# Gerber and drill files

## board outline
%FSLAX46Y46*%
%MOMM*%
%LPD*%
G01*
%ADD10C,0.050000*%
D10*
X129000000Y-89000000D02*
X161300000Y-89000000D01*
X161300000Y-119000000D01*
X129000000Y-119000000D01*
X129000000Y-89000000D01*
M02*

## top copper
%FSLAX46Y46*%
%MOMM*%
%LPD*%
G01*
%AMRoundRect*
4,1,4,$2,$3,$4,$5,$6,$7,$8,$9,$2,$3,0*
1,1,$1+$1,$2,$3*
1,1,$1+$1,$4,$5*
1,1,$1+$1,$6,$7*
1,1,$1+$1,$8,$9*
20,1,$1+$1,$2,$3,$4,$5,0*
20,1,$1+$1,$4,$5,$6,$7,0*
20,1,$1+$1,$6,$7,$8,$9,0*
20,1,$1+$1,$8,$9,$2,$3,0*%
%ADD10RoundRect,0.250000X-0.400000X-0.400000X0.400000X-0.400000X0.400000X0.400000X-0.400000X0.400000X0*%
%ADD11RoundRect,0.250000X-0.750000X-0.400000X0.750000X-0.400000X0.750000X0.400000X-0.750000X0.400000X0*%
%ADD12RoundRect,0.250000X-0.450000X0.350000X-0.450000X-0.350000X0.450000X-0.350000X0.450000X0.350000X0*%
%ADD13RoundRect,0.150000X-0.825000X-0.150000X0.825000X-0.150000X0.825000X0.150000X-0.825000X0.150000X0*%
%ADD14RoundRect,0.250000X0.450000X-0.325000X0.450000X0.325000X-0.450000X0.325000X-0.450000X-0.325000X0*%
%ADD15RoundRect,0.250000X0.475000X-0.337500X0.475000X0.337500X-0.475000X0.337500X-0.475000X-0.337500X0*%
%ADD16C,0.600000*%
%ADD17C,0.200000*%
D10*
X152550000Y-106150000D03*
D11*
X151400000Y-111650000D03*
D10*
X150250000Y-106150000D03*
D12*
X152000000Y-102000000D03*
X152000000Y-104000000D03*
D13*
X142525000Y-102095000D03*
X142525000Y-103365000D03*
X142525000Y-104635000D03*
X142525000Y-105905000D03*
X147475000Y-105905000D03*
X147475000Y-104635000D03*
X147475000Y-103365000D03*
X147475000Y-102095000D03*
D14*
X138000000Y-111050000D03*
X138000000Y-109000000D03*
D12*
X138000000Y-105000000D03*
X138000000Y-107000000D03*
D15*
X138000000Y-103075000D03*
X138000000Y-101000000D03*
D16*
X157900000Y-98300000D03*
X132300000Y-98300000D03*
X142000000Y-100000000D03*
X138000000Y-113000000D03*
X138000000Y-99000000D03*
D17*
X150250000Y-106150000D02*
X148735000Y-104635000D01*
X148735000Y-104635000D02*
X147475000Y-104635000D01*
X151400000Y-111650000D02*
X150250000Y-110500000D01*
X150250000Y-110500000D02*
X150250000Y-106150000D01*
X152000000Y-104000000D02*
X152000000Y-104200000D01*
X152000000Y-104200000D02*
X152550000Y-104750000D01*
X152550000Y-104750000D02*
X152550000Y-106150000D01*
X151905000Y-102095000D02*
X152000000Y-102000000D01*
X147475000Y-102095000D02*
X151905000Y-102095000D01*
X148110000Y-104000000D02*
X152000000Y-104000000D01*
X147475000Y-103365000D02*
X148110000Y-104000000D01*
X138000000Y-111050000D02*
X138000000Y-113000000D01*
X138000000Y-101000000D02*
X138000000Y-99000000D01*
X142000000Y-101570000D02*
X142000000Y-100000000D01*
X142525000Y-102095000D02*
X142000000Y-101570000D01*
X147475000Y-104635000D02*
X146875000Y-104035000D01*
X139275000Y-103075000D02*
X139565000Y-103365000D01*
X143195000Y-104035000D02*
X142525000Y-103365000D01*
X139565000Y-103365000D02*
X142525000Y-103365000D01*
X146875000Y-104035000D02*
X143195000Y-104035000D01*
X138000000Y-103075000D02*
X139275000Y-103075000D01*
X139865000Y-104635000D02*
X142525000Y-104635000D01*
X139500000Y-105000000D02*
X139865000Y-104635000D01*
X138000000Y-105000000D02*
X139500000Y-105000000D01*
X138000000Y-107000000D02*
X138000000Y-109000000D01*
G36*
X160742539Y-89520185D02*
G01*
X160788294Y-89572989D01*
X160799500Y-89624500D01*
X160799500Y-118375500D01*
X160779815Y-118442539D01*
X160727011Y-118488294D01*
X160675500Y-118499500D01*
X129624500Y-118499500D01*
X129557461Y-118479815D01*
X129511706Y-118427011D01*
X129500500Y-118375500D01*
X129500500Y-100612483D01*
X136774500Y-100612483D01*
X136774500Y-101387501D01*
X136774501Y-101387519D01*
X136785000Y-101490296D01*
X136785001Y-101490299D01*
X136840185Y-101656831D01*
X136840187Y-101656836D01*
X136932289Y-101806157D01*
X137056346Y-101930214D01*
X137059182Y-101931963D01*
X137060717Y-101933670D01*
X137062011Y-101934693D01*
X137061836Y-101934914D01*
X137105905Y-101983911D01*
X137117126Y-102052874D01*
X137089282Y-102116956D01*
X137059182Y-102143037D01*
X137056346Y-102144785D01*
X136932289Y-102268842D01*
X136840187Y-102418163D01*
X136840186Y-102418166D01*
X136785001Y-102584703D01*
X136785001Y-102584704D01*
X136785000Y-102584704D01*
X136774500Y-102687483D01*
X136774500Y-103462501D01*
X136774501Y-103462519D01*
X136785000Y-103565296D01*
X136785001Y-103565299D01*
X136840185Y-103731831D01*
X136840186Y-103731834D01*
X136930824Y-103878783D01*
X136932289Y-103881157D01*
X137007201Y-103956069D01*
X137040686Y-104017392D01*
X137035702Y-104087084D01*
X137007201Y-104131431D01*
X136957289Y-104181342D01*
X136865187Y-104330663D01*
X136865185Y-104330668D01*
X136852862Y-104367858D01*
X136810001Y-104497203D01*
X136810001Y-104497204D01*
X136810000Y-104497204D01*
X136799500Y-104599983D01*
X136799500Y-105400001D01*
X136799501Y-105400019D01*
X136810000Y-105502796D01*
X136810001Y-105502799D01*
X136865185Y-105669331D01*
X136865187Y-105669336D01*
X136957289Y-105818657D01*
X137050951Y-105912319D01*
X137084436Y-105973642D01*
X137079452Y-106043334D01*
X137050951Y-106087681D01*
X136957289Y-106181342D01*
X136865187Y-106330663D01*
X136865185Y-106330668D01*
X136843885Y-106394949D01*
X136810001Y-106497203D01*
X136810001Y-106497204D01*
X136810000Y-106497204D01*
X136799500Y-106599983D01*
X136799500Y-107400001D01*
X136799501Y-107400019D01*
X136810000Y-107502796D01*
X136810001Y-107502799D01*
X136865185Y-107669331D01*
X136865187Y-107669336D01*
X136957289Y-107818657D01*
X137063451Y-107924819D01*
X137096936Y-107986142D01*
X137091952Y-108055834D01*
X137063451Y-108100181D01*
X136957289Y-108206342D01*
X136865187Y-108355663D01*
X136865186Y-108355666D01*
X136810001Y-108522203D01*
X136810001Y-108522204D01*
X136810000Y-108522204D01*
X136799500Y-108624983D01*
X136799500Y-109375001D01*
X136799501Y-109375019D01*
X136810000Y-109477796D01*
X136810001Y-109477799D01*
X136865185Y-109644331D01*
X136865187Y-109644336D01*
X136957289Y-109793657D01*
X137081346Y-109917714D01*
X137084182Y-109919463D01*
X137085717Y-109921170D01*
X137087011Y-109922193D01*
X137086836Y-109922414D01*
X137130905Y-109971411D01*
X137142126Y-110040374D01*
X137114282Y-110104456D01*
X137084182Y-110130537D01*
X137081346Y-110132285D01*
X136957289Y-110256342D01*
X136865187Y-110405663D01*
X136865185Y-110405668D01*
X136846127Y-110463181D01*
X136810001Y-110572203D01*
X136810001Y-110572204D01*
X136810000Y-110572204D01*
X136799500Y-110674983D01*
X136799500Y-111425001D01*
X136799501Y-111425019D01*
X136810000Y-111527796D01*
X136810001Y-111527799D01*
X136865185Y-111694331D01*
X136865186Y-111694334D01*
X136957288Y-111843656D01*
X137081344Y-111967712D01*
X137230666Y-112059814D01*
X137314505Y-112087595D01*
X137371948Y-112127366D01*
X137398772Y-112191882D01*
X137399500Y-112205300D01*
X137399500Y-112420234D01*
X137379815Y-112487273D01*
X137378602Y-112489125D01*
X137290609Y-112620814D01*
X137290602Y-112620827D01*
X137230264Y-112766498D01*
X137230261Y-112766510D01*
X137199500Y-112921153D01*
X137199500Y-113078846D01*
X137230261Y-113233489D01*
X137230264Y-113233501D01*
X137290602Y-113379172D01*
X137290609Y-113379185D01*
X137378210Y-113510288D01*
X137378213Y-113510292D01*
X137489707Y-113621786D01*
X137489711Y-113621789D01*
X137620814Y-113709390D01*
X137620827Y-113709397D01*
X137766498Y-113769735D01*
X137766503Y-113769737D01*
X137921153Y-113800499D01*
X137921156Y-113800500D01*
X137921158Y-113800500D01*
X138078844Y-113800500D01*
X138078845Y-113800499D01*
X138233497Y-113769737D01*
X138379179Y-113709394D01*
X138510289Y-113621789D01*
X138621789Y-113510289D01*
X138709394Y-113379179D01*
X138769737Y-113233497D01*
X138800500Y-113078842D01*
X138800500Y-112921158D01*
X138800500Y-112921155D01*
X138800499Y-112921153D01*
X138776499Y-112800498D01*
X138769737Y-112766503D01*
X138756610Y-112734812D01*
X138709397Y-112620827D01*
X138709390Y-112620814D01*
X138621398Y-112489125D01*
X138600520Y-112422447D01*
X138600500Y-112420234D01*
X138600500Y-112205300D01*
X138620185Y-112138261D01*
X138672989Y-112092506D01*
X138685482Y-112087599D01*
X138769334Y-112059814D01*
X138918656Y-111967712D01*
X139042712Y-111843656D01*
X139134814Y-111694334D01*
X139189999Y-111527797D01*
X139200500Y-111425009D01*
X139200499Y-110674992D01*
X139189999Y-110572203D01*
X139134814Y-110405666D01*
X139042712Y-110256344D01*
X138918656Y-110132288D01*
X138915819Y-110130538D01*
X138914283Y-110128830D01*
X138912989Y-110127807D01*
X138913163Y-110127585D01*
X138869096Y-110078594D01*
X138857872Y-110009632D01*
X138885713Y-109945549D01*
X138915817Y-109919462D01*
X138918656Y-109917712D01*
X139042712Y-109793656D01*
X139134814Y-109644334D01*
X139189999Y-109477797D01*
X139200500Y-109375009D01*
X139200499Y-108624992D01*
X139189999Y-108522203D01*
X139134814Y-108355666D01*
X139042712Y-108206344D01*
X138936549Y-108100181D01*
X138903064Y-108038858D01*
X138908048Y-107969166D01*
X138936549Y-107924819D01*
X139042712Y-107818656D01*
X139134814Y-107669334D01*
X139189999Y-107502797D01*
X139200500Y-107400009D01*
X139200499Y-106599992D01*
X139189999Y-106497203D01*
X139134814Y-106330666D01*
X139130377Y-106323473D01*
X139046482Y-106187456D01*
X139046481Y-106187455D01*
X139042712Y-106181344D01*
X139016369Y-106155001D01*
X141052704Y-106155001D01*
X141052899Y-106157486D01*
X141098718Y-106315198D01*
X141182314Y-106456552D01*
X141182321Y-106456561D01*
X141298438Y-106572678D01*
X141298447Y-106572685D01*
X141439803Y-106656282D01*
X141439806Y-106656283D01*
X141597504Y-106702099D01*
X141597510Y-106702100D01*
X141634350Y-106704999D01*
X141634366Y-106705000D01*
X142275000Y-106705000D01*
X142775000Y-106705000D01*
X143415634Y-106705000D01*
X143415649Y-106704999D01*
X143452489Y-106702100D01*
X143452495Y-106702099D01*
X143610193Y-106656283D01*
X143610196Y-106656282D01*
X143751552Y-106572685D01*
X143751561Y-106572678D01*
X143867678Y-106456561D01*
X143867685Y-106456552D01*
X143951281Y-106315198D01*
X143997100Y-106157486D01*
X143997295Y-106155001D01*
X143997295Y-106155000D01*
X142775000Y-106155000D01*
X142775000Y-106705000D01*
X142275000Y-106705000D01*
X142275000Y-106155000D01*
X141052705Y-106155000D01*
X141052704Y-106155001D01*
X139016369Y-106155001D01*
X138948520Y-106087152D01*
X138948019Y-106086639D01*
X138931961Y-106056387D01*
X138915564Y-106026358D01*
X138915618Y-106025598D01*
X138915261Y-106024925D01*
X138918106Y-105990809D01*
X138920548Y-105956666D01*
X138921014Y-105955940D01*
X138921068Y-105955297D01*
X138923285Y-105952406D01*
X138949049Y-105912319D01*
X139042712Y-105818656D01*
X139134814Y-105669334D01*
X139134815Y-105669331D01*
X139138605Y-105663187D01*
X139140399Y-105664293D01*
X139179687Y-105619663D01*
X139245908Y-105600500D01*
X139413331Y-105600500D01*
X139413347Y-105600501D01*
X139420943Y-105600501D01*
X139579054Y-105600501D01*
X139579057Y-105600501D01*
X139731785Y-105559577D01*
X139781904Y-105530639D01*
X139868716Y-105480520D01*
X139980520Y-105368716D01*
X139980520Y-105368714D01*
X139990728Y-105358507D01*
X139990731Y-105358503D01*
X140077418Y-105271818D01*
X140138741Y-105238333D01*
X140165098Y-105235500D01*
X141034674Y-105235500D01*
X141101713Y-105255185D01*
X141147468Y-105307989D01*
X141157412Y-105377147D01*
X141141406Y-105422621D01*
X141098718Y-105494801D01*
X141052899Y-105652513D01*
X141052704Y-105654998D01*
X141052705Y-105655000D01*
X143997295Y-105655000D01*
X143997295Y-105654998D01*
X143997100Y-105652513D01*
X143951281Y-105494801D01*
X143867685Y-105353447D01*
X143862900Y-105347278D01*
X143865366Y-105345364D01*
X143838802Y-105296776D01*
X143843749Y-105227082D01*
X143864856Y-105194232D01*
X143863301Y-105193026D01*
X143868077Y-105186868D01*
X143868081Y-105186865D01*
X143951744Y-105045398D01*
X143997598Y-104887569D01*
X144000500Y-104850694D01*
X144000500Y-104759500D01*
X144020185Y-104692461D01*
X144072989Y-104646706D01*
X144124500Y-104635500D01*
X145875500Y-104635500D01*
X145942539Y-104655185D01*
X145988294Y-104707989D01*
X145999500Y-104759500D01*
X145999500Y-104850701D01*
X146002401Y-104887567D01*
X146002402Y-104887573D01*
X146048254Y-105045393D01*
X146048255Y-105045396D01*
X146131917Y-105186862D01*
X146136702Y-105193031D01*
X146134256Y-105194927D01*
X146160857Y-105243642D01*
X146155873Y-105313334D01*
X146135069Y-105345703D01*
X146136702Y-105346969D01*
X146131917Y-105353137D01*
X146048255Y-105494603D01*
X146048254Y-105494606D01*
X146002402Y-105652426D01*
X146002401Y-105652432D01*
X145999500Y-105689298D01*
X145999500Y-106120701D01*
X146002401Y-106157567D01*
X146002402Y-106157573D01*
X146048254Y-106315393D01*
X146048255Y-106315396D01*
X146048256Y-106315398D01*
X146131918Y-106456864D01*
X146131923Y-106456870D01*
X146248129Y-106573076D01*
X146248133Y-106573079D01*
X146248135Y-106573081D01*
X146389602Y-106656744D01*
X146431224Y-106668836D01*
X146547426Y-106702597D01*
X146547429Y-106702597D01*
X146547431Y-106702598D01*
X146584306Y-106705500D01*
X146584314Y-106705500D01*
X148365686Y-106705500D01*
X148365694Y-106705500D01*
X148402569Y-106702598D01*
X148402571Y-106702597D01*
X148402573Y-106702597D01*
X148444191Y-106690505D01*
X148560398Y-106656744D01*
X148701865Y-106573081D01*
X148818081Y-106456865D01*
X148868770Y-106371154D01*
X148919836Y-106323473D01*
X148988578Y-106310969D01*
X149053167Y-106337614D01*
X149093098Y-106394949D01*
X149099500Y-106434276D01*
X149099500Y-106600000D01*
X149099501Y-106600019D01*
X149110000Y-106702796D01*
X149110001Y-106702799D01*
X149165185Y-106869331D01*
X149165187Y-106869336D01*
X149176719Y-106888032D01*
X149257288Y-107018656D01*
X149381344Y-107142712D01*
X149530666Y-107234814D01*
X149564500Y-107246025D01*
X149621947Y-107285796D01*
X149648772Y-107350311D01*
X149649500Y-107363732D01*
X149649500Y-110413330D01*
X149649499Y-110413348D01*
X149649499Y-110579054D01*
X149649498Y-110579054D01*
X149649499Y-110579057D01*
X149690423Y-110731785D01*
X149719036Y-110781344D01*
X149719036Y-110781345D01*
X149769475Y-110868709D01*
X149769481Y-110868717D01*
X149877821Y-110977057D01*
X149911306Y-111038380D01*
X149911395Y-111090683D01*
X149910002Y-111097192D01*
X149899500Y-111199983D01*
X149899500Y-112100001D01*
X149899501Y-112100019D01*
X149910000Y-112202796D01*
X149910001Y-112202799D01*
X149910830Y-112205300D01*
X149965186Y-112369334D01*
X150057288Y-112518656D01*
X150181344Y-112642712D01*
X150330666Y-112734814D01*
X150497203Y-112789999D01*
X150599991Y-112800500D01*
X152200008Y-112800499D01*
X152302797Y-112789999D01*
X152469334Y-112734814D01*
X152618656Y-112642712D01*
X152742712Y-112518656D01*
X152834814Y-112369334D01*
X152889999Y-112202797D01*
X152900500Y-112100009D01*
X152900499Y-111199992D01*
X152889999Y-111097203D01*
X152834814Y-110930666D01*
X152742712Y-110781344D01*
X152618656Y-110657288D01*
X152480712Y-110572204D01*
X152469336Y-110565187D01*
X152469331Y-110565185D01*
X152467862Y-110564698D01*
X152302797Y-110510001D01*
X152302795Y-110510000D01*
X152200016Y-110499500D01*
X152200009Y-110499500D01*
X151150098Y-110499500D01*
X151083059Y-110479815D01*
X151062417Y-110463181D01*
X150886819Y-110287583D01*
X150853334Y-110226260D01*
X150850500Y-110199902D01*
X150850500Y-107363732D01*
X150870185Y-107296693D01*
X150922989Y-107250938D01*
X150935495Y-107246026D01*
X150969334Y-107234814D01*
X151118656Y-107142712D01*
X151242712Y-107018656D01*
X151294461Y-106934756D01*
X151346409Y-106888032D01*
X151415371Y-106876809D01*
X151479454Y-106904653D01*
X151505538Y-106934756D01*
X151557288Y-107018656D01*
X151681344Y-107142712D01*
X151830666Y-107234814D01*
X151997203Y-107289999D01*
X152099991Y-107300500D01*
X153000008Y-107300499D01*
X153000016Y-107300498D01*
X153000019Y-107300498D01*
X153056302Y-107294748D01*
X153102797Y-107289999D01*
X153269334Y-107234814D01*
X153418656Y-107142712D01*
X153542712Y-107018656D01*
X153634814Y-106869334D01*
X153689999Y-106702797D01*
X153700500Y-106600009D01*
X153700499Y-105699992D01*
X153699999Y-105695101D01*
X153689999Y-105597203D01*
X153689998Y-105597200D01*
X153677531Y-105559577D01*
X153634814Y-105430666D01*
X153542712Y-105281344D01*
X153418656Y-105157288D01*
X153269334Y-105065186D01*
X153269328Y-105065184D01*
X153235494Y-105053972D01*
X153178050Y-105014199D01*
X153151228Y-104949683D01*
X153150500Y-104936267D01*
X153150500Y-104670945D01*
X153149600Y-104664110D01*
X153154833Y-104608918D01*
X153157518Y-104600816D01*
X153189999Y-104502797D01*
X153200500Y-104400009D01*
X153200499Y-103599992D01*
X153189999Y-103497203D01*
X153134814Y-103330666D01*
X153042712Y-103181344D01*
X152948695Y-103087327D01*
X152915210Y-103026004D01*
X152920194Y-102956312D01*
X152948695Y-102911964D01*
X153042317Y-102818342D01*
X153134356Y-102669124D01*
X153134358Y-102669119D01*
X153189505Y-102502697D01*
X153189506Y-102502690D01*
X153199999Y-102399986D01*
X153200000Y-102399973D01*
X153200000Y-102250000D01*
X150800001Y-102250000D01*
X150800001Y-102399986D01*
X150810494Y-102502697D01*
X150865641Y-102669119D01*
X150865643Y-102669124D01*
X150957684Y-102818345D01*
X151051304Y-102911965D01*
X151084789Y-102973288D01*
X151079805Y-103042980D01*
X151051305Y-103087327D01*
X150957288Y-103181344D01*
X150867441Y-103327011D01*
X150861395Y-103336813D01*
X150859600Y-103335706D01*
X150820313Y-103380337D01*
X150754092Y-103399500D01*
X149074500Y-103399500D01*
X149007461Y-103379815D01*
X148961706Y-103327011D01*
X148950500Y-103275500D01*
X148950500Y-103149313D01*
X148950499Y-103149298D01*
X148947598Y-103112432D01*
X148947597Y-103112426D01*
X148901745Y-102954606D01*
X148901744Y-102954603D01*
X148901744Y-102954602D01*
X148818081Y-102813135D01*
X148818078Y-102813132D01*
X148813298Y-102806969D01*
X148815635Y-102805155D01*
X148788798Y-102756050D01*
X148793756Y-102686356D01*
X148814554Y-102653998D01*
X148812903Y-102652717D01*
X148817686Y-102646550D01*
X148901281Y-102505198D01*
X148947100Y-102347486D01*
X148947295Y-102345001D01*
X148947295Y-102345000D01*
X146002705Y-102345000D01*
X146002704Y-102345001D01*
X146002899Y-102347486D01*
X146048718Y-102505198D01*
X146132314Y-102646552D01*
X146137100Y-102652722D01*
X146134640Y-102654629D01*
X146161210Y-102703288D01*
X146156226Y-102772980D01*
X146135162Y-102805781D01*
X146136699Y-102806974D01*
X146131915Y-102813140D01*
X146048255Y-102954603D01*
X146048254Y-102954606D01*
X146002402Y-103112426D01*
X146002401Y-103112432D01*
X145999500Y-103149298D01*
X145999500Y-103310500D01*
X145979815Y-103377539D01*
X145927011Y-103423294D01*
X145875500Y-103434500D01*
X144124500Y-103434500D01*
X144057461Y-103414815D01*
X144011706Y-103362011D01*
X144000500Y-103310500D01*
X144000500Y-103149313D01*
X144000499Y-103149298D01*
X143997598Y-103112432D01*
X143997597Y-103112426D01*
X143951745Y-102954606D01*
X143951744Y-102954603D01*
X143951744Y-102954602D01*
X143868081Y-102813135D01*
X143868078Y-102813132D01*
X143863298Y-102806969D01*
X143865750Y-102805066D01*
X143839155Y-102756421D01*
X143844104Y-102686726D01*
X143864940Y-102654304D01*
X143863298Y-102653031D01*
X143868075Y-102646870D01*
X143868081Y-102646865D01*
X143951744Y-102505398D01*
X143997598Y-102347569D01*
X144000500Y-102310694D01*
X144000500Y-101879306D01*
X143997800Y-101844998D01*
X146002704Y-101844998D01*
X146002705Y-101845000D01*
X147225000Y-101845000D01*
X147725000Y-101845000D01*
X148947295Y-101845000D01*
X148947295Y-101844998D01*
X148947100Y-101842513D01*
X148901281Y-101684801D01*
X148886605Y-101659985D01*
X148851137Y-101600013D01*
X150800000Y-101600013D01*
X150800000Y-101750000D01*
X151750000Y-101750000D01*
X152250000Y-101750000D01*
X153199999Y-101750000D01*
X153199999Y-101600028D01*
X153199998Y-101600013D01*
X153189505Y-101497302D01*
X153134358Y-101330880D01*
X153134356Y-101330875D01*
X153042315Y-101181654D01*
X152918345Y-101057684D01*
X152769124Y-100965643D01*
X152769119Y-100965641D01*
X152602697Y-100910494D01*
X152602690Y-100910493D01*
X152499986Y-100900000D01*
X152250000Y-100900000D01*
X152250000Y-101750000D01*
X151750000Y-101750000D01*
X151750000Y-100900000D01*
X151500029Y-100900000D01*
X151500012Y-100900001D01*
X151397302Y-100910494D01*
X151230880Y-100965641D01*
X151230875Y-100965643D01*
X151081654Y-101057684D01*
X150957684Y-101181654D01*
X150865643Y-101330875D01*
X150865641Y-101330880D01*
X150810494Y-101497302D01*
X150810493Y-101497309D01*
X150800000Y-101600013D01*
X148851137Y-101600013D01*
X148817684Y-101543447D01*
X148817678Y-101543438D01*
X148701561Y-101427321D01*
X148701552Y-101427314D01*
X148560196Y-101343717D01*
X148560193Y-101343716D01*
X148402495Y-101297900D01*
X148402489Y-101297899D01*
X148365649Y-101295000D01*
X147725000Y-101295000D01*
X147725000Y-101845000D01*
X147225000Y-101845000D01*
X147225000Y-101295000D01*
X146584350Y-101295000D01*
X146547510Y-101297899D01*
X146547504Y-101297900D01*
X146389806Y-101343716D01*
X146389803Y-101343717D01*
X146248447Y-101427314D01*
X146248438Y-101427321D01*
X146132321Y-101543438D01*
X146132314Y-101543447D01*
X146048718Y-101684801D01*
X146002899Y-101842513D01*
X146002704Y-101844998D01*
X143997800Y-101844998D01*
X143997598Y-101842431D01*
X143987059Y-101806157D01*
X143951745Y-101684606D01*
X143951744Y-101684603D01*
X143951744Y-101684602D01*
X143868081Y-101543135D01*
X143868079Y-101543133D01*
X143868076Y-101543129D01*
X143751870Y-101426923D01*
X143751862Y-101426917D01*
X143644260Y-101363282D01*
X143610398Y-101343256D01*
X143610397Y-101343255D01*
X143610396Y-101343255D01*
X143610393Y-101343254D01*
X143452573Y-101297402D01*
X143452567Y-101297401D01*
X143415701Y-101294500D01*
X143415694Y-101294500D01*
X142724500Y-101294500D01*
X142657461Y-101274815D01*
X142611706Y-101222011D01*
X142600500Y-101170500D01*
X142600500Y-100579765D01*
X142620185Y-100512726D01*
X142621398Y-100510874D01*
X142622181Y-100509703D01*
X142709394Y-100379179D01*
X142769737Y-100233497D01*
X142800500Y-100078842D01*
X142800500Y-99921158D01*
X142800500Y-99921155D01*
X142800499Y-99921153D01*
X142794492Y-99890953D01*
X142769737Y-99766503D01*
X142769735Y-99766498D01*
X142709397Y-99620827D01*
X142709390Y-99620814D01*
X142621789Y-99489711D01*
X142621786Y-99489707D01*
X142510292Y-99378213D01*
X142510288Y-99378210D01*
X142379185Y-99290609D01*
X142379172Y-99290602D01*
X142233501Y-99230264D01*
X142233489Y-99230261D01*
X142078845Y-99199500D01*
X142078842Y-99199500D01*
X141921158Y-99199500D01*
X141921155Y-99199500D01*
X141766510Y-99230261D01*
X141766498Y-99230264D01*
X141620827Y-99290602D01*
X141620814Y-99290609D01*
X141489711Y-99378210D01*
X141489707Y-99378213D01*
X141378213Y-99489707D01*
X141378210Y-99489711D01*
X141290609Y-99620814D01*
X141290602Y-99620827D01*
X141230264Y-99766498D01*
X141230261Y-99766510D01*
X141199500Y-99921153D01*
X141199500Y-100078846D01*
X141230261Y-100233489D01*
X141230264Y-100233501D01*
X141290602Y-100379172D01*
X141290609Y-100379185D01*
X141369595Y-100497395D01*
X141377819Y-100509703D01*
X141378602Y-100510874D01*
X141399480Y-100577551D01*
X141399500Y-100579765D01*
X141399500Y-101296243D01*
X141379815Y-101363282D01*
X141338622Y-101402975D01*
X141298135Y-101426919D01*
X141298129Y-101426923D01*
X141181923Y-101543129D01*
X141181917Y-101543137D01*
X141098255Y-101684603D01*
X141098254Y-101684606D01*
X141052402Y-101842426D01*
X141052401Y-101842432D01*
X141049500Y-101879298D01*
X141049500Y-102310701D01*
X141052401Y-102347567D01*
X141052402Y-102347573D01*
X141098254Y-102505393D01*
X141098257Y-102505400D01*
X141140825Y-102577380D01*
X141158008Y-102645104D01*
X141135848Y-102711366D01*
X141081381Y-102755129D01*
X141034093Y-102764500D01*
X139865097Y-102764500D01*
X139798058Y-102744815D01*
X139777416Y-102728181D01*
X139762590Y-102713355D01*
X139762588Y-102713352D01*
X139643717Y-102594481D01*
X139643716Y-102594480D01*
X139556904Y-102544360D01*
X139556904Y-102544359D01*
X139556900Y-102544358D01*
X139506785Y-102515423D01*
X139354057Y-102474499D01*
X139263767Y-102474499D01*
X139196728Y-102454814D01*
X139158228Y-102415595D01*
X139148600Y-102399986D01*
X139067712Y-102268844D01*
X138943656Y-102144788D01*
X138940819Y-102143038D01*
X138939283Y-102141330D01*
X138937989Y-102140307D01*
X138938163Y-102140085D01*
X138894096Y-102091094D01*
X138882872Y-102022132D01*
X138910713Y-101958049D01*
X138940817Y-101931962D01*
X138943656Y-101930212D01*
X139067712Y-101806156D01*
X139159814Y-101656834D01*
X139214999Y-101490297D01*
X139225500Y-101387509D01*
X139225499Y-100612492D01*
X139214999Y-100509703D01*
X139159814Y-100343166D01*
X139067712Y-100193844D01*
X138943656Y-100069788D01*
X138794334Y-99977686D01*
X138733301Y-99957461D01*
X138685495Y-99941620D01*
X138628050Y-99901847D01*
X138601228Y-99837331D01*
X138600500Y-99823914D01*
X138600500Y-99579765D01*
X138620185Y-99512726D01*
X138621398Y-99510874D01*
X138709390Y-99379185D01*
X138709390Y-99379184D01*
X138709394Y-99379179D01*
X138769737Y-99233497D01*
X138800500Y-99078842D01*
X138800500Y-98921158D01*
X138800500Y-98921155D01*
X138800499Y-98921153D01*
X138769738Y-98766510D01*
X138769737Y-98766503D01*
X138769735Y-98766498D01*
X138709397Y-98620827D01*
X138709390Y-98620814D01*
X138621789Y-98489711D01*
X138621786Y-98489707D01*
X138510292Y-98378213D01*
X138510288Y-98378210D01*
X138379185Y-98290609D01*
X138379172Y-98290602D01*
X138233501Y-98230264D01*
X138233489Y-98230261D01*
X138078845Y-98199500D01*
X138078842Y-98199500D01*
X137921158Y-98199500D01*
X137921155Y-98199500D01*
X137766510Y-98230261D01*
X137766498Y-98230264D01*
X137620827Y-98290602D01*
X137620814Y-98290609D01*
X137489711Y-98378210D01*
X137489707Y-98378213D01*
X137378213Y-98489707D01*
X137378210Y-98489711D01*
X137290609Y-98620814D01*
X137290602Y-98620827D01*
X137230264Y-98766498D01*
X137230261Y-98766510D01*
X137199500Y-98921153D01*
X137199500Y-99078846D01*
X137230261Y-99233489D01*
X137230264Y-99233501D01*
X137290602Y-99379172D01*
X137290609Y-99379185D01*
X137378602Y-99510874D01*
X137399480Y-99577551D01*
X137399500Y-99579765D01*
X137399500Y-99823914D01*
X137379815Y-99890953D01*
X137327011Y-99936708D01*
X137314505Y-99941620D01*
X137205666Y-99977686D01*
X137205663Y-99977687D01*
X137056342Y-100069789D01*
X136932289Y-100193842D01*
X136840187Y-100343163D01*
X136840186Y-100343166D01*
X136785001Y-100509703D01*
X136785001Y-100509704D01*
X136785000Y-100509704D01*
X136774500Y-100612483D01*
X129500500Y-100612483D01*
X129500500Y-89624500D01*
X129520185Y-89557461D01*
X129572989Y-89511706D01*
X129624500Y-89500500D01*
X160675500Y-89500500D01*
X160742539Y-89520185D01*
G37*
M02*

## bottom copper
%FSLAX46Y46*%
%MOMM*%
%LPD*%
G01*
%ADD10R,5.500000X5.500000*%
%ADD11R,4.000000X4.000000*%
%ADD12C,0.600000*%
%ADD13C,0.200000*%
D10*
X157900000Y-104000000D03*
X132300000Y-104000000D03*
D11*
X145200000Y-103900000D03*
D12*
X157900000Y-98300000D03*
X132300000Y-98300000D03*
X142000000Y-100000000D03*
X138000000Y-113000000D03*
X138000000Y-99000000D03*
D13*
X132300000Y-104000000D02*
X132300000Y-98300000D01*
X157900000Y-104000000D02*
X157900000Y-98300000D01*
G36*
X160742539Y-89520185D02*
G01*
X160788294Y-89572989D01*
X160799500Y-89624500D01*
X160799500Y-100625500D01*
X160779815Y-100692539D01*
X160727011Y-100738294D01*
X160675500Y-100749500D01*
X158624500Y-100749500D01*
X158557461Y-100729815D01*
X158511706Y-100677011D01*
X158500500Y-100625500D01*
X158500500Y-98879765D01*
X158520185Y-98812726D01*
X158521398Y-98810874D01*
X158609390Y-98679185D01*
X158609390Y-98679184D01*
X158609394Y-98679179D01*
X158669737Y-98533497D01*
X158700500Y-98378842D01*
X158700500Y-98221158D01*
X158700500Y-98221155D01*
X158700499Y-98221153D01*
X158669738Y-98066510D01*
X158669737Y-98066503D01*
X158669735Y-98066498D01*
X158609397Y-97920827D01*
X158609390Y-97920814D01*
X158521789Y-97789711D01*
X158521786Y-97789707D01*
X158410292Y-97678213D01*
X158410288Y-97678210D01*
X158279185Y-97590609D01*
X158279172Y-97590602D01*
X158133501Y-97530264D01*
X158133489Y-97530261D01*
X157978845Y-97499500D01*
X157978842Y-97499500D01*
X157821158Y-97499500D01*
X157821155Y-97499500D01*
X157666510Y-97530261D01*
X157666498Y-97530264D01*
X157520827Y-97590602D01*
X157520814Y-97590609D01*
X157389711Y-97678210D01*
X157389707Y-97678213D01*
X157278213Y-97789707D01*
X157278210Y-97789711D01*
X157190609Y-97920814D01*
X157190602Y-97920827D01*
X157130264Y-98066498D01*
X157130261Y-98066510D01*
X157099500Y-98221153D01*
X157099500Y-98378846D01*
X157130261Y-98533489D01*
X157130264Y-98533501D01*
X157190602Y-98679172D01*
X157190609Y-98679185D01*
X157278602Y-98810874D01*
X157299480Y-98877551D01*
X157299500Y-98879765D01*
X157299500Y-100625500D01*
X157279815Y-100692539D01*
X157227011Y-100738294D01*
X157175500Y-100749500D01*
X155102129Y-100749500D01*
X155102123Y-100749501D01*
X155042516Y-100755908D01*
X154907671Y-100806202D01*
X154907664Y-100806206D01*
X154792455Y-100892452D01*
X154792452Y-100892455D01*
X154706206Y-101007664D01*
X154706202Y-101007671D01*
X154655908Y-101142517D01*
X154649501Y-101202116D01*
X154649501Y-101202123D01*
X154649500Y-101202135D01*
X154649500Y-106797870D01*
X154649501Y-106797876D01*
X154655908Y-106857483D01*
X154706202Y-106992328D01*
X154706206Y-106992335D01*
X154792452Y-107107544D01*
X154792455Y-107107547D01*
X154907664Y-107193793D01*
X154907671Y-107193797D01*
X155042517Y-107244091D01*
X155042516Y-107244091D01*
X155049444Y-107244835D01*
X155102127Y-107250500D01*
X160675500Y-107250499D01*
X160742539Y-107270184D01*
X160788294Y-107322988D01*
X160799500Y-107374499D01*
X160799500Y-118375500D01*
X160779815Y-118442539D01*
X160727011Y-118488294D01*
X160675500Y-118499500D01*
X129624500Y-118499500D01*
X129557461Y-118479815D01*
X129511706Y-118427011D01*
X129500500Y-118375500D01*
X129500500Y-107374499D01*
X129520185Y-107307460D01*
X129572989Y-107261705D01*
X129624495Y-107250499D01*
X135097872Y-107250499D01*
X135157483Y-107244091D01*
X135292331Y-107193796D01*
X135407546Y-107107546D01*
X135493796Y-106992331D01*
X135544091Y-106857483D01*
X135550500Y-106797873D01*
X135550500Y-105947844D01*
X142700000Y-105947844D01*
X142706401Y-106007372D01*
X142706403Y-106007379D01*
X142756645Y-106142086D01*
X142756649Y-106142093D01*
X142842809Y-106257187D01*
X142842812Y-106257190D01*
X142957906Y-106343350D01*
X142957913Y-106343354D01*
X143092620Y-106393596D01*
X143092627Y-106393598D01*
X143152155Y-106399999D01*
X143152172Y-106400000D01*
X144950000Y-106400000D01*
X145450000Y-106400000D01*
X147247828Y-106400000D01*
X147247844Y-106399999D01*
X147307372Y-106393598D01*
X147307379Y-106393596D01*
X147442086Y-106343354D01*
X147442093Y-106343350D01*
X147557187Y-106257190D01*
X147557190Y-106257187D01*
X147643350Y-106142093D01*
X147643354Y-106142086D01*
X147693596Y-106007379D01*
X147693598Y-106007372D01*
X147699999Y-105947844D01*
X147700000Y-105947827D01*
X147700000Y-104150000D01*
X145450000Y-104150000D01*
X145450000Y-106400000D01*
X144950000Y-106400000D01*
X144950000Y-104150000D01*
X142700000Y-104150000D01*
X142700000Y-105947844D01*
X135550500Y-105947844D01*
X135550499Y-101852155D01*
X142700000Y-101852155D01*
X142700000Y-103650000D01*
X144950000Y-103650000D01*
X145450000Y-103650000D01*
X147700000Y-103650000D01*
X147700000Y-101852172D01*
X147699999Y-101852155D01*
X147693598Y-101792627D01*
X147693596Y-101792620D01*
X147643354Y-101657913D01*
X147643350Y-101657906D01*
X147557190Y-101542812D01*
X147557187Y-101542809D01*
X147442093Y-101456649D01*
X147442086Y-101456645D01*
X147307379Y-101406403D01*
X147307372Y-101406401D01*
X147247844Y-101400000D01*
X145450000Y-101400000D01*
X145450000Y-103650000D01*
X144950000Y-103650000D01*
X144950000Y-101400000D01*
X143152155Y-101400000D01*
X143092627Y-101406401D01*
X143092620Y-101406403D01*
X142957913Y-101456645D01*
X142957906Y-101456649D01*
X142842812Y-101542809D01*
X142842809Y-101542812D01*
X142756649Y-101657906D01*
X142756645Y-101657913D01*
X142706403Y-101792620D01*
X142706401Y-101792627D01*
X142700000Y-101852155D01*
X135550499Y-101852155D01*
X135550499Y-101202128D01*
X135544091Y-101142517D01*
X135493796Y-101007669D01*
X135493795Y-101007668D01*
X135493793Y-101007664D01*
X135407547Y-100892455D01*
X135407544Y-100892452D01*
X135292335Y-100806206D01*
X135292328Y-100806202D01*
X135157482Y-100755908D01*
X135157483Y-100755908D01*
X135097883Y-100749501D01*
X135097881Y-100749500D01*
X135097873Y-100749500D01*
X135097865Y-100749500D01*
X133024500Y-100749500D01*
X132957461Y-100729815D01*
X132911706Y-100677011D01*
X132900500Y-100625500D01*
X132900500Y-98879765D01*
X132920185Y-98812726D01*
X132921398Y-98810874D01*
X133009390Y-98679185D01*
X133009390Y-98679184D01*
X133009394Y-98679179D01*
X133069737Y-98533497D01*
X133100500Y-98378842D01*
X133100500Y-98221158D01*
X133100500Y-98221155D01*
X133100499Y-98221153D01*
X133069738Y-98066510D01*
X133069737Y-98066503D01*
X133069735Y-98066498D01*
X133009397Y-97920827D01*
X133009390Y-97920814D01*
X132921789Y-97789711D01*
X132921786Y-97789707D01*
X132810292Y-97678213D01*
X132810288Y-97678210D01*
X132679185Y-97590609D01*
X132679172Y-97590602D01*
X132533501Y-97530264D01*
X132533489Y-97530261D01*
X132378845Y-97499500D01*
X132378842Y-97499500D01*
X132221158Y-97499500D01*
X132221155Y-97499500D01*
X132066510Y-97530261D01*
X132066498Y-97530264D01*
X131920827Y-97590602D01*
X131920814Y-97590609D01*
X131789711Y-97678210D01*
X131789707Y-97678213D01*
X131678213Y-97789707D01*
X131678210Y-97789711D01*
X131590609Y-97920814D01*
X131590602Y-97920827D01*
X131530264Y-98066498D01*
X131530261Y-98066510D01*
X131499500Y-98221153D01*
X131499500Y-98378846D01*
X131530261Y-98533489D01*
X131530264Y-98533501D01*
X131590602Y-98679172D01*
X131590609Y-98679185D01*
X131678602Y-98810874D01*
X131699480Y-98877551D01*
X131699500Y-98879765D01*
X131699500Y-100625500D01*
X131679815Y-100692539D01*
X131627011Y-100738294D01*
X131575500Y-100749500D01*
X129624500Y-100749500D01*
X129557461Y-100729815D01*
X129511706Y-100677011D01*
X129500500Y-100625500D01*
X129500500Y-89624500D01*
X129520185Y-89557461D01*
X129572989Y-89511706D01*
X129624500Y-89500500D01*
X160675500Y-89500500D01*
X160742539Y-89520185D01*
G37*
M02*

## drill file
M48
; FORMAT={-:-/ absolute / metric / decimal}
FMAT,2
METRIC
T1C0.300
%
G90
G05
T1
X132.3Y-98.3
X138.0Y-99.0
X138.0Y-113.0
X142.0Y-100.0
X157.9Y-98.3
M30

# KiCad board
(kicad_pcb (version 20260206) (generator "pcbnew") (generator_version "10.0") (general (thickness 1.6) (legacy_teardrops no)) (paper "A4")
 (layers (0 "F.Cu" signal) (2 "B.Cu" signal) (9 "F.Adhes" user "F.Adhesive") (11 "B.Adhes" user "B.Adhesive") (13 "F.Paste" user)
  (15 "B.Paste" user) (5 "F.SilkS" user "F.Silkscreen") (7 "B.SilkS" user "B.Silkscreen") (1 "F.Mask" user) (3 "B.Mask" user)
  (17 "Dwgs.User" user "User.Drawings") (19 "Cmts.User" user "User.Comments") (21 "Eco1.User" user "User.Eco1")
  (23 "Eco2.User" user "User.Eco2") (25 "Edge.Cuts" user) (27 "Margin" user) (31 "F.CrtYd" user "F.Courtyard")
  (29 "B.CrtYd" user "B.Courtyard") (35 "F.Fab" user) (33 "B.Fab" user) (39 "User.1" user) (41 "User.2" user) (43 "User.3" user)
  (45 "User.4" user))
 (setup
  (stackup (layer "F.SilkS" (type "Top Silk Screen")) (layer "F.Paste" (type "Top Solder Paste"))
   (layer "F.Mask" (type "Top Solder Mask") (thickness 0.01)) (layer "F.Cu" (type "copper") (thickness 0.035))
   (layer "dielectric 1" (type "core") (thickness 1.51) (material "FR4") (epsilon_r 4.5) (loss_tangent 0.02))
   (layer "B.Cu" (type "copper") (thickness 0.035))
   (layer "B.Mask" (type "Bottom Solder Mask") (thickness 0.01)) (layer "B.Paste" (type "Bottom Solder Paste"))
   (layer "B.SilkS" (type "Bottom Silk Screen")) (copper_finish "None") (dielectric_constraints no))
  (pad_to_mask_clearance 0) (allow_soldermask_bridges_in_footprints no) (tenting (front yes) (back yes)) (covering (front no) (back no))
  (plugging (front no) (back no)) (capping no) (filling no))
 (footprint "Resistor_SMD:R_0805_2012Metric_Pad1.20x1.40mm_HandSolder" (layer "F.Cu") (at 152 103 -90)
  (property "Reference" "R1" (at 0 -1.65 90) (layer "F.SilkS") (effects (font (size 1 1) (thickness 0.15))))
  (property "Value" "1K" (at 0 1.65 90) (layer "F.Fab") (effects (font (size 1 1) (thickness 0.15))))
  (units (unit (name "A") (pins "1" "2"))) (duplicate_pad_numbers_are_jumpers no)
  (pad "1" smd roundrect (at -1 0 270) (size 1.2 1.4) (layers "F.Cu" "F.Mask" "F.Paste") (roundrect_rratio 0.208333) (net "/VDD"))
  (pad "2" smd roundrect (at 1 0 270) (size 1.2 1.4) (layers "F.Cu" "F.Mask" "F.Paste") (roundrect_rratio 0.208333) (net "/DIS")))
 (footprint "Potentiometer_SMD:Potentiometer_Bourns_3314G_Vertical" (layer "F.Cu") (at 151.4 108.9)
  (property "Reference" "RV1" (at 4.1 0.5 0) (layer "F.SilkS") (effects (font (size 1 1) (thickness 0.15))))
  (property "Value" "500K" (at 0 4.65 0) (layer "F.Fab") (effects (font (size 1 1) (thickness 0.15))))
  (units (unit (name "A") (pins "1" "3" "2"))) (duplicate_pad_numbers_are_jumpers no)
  (pad "1" smd roundrect (at 1.15 -2.75) (size 1.3 1.3) (layers "F.Cu" "F.Mask" "F.Paste") (roundrect_rratio 0.192308) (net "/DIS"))
  (pad "2" smd roundrect (at 0 2.75) (size 2 1.3) (layers "F.Cu" "F.Mask" "F.Paste") (roundrect_rratio 0.192308) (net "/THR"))
  (pad "3" smd roundrect (at -1.15 -2.75) (size 1.3 1.3) (layers "F.Cu" "F.Mask" "F.Paste") (roundrect_rratio 0.192308) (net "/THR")))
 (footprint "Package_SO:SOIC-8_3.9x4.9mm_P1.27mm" (layer "F.Cu") (at 145 104)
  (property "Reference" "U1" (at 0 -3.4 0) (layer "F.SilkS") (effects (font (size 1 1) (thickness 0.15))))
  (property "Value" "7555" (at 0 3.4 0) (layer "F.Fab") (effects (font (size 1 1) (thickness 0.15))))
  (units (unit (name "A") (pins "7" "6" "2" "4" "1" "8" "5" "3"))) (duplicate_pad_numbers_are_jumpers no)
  (pad "1" smd roundrect (at -2.475 -1.905) (size 1.95 0.6) (layers "F.Cu" "F.Mask" "F.Paste") (roundrect_rratio 0.25) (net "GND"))
  (pad "2" smd roundrect (at -2.475 -0.635) (size 1.95 0.6) (layers "F.Cu" "F.Mask" "F.Paste") (roundrect_rratio 0.25) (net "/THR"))
  (pad "3" smd roundrect (at -2.475 0.635) (size 1.95 0.6) (layers "F.Cu" "F.Mask" "F.Paste") (roundrect_rratio 0.25) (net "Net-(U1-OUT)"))
  (pad "4" smd roundrect (at -2.475 1.905) (size 1.95 0.6) (layers "F.Cu" "F.Mask" "F.Paste") (roundrect_rratio 0.25) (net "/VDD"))
  (pad "5" smd roundrect (at 2.475 1.905) (size 1.95 0.6) (layers "F.Cu" "F.Mask" "F.Paste") (roundrect_rratio 0.25)
   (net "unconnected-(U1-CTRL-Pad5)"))
  (pad "6" smd roundrect (at 2.475 0.635) (size 1.95 0.6) (layers "F.Cu" "F.Mask" "F.Paste") (roundrect_rratio 0.25) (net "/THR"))
  (pad "7" smd roundrect (at 2.475 -0.635) (size 1.95 0.6) (layers "F.Cu" "F.Mask" "F.Paste") (roundrect_rratio 0.25) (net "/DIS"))
  (pad "8" smd roundrect (at 2.475 -1.905) (size 1.95 0.6) (layers "F.Cu" "F.Mask" "F.Paste") (roundrect_rratio 0.25) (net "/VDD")))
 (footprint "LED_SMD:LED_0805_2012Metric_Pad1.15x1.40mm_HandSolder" (layer "F.Cu") (at 138 110.025 90)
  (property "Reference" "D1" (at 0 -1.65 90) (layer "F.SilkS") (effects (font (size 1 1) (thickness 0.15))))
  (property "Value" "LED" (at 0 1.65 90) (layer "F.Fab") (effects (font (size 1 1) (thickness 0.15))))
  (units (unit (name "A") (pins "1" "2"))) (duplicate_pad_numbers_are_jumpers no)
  (pad "1" smd roundrect (at -1.025 0 90) (size 1.15 1.4) (layers "F.Cu" "F.Mask" "F.Paste") (roundrect_rratio 0.217391) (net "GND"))
  (pad "2" smd roundrect (at 1.025 0 90) (size 1.15 1.4) (layers "F.Cu" "F.Mask" "F.Paste") (roundrect_rratio 0.217391) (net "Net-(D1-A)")))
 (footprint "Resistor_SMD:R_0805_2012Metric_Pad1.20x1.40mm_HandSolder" (layer "F.Cu") (at 138 106 -90)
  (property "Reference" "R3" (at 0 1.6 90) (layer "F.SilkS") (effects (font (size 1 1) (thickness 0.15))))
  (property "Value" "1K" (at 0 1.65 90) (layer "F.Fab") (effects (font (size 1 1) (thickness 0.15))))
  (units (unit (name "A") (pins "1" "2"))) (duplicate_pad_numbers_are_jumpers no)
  (pad "1" smd roundrect (at -1 0 270) (size 1.2 1.4) (layers "F.Cu" "F.Mask" "F.Paste") (roundrect_rratio 0.208333) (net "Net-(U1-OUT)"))
  (pad "2" smd roundrect (at 1 0 270) (size 1.2 1.4) (layers "F.Cu" "F.Mask" "F.Paste") (roundrect_rratio 0.208333) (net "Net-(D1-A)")))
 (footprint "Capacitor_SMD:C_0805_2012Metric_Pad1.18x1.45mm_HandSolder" (layer "F.Cu") (at 138 102.0375 90)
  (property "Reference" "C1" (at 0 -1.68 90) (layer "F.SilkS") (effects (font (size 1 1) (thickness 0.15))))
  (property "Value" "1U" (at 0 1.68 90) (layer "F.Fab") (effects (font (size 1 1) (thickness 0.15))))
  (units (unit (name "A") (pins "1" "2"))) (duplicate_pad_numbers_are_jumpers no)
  (pad "1" smd roundrect (at -1.0375 0 90) (size 1.175 1.45) (layers "F.Cu" "F.Mask" "F.Paste") (roundrect_rratio 0.212766) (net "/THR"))
  (pad "2" smd roundrect (at 1.0375 0 90) (size 1.175 1.45) (layers "F.Cu" "F.Mask" "F.Paste") (roundrect_rratio 0.212766) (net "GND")))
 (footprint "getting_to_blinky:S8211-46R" (layer "B.Cu") (at 145.1 104 180)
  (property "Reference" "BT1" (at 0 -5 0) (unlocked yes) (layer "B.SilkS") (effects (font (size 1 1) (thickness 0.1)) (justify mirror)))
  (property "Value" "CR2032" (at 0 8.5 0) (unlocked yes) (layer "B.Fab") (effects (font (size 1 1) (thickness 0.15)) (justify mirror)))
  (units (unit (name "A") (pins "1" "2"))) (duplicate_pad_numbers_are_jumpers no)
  (pad "1" smd rect (at -12.8 0 180) (size 5.5 5.5) (layers "B.Cu" "B.Mask" "B.Paste") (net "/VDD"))
  (pad "1" smd rect (at 12.8 0 180) (size 5.5 5.5) (layers "B.Cu" "B.Mask" "B.Paste") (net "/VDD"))
  (pad "2" smd rect (at -0.1 0.1 180) (size 4 4) (layers "B.Cu" "B.Mask" "B.Paste") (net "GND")))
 (gr_rect (start 129 89) (end 161.3 119) (stroke (width 0.05) (type default)) (fill no) (layer "Edge.Cuts"))
 (segment (start 151.905 102.095) (end 152 102) (width 0.2) (layer "F.Cu") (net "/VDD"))
 (segment (start 147.475 102.095) (end 151.905 102.095) (width 0.2) (layer "F.Cu") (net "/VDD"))
 (via (at 157.9 98.3) (size 0.6) (drill 0.3) (layers "F.Cu" "B.Cu") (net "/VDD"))
 (via (at 132.3 98.3) (size 0.6) (drill 0.3) (layers "F.Cu" "B.Cu") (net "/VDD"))
 (segment (start 132.3 104) (end 132.3 98.3) (width 0.2) (layer "B.Cu") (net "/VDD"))
 (segment (start 157.9 104) (end 157.9 98.3) (width 0.2) (layer "B.Cu") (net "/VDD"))
 (segment (start 152 104.2) (end 152.55 104.75) (width 0.2) (layer "F.Cu") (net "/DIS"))
 (segment (start 148.11 104) (end 152 104) (width 0.2) (layer "F.Cu") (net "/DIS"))
 (segment (start 152 104) (end 152 104.2) (width 0.2) (layer "F.Cu") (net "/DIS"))
 (segment (start 152.55 104.75) (end 152.55 106.15) (width 0.2) (layer "F.Cu") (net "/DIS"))
 (segment (start 147.475 103.365) (end 148.11 104) (width 0.2) (layer "F.Cu") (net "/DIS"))
 (segment (start 138 111.05) (end 138 113) (width 0.2) (layer "F.Cu") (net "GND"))
 (segment (start 138 101) (end 138 99) (width 0.2) (layer "F.Cu") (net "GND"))
 (segment (start 142 101.57) (end 142 100) (width 0.2) (layer "F.Cu") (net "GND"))
 (segment (start 142.525 102.095) (end 142 101.57) (width 0.2) (layer "F.Cu") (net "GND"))
 (via (at 142 100) (size 0.6) (drill 0.3) (layers "F.Cu" "B.Cu") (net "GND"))
 (via (at 138 113) (size 0.6) (drill 0.3) (layers "F.Cu" "B.Cu") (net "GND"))
 (via (at 138 99) (size 0.6) (drill 0.3) (layers "F.Cu" "B.Cu") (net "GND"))
 (segment (start 150.25 106.15) (end 148.735 104.635) (width 0.2) (layer "F.Cu") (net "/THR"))
 (segment (start 147.475 104.635) (end 146.875 104.035) (width 0.2) (layer "F.Cu") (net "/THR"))
 (segment (start 150.25 110.5) (end 150.25 106.15) (width 0.2) (layer "F.Cu") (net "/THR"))
 (segment (start 139.275 103.075) (end 139.565 103.365) (width 0.2) (layer "F.Cu") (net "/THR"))
 (segment (start 143.195 104.035) (end 142.525 103.365) (width 0.2) (layer "F.Cu") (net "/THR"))
 (segment (start 148.735 104.635) (end 147.475 104.635) (width 0.2) (layer "F.Cu") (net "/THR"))
 (segment (start 139.565 103.365) (end 142.525 103.365) (width 0.2) (layer "F.Cu") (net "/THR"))
 (segment (start 146.875 104.035) (end 143.195 104.035) (width 0.2) (layer "F.Cu") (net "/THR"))
 (segment (start 138 103.075) (end 139.275 103.075) (width 0.2) (layer "F.Cu") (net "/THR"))
 (segment (start 151.4 111.65) (end 150.25 110.5) (width 0.2) (layer "F.Cu") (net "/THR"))
 (segment (start 139.865 104.635) (end 142.525 104.635) (width 0.2) (layer "F.Cu") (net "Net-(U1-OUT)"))
 (segment (start 139.5 105) (end 139.865 104.635) (width 0.2) (layer "F.Cu") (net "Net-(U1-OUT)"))
 (segment (start 138 105) (end 139.5 105) (width 0.2) (layer "F.Cu") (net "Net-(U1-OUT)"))
 (segment (start 138 107) (end 138 109) (width 0.2) (layer "F.Cu") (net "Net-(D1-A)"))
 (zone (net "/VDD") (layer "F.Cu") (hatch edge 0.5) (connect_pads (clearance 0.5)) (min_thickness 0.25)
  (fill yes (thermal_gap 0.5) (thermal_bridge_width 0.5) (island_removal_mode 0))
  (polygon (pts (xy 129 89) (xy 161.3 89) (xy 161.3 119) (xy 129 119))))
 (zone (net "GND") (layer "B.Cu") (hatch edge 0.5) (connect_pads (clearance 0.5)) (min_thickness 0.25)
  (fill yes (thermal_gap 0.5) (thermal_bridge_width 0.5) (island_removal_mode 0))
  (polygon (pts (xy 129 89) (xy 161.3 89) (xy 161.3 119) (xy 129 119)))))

